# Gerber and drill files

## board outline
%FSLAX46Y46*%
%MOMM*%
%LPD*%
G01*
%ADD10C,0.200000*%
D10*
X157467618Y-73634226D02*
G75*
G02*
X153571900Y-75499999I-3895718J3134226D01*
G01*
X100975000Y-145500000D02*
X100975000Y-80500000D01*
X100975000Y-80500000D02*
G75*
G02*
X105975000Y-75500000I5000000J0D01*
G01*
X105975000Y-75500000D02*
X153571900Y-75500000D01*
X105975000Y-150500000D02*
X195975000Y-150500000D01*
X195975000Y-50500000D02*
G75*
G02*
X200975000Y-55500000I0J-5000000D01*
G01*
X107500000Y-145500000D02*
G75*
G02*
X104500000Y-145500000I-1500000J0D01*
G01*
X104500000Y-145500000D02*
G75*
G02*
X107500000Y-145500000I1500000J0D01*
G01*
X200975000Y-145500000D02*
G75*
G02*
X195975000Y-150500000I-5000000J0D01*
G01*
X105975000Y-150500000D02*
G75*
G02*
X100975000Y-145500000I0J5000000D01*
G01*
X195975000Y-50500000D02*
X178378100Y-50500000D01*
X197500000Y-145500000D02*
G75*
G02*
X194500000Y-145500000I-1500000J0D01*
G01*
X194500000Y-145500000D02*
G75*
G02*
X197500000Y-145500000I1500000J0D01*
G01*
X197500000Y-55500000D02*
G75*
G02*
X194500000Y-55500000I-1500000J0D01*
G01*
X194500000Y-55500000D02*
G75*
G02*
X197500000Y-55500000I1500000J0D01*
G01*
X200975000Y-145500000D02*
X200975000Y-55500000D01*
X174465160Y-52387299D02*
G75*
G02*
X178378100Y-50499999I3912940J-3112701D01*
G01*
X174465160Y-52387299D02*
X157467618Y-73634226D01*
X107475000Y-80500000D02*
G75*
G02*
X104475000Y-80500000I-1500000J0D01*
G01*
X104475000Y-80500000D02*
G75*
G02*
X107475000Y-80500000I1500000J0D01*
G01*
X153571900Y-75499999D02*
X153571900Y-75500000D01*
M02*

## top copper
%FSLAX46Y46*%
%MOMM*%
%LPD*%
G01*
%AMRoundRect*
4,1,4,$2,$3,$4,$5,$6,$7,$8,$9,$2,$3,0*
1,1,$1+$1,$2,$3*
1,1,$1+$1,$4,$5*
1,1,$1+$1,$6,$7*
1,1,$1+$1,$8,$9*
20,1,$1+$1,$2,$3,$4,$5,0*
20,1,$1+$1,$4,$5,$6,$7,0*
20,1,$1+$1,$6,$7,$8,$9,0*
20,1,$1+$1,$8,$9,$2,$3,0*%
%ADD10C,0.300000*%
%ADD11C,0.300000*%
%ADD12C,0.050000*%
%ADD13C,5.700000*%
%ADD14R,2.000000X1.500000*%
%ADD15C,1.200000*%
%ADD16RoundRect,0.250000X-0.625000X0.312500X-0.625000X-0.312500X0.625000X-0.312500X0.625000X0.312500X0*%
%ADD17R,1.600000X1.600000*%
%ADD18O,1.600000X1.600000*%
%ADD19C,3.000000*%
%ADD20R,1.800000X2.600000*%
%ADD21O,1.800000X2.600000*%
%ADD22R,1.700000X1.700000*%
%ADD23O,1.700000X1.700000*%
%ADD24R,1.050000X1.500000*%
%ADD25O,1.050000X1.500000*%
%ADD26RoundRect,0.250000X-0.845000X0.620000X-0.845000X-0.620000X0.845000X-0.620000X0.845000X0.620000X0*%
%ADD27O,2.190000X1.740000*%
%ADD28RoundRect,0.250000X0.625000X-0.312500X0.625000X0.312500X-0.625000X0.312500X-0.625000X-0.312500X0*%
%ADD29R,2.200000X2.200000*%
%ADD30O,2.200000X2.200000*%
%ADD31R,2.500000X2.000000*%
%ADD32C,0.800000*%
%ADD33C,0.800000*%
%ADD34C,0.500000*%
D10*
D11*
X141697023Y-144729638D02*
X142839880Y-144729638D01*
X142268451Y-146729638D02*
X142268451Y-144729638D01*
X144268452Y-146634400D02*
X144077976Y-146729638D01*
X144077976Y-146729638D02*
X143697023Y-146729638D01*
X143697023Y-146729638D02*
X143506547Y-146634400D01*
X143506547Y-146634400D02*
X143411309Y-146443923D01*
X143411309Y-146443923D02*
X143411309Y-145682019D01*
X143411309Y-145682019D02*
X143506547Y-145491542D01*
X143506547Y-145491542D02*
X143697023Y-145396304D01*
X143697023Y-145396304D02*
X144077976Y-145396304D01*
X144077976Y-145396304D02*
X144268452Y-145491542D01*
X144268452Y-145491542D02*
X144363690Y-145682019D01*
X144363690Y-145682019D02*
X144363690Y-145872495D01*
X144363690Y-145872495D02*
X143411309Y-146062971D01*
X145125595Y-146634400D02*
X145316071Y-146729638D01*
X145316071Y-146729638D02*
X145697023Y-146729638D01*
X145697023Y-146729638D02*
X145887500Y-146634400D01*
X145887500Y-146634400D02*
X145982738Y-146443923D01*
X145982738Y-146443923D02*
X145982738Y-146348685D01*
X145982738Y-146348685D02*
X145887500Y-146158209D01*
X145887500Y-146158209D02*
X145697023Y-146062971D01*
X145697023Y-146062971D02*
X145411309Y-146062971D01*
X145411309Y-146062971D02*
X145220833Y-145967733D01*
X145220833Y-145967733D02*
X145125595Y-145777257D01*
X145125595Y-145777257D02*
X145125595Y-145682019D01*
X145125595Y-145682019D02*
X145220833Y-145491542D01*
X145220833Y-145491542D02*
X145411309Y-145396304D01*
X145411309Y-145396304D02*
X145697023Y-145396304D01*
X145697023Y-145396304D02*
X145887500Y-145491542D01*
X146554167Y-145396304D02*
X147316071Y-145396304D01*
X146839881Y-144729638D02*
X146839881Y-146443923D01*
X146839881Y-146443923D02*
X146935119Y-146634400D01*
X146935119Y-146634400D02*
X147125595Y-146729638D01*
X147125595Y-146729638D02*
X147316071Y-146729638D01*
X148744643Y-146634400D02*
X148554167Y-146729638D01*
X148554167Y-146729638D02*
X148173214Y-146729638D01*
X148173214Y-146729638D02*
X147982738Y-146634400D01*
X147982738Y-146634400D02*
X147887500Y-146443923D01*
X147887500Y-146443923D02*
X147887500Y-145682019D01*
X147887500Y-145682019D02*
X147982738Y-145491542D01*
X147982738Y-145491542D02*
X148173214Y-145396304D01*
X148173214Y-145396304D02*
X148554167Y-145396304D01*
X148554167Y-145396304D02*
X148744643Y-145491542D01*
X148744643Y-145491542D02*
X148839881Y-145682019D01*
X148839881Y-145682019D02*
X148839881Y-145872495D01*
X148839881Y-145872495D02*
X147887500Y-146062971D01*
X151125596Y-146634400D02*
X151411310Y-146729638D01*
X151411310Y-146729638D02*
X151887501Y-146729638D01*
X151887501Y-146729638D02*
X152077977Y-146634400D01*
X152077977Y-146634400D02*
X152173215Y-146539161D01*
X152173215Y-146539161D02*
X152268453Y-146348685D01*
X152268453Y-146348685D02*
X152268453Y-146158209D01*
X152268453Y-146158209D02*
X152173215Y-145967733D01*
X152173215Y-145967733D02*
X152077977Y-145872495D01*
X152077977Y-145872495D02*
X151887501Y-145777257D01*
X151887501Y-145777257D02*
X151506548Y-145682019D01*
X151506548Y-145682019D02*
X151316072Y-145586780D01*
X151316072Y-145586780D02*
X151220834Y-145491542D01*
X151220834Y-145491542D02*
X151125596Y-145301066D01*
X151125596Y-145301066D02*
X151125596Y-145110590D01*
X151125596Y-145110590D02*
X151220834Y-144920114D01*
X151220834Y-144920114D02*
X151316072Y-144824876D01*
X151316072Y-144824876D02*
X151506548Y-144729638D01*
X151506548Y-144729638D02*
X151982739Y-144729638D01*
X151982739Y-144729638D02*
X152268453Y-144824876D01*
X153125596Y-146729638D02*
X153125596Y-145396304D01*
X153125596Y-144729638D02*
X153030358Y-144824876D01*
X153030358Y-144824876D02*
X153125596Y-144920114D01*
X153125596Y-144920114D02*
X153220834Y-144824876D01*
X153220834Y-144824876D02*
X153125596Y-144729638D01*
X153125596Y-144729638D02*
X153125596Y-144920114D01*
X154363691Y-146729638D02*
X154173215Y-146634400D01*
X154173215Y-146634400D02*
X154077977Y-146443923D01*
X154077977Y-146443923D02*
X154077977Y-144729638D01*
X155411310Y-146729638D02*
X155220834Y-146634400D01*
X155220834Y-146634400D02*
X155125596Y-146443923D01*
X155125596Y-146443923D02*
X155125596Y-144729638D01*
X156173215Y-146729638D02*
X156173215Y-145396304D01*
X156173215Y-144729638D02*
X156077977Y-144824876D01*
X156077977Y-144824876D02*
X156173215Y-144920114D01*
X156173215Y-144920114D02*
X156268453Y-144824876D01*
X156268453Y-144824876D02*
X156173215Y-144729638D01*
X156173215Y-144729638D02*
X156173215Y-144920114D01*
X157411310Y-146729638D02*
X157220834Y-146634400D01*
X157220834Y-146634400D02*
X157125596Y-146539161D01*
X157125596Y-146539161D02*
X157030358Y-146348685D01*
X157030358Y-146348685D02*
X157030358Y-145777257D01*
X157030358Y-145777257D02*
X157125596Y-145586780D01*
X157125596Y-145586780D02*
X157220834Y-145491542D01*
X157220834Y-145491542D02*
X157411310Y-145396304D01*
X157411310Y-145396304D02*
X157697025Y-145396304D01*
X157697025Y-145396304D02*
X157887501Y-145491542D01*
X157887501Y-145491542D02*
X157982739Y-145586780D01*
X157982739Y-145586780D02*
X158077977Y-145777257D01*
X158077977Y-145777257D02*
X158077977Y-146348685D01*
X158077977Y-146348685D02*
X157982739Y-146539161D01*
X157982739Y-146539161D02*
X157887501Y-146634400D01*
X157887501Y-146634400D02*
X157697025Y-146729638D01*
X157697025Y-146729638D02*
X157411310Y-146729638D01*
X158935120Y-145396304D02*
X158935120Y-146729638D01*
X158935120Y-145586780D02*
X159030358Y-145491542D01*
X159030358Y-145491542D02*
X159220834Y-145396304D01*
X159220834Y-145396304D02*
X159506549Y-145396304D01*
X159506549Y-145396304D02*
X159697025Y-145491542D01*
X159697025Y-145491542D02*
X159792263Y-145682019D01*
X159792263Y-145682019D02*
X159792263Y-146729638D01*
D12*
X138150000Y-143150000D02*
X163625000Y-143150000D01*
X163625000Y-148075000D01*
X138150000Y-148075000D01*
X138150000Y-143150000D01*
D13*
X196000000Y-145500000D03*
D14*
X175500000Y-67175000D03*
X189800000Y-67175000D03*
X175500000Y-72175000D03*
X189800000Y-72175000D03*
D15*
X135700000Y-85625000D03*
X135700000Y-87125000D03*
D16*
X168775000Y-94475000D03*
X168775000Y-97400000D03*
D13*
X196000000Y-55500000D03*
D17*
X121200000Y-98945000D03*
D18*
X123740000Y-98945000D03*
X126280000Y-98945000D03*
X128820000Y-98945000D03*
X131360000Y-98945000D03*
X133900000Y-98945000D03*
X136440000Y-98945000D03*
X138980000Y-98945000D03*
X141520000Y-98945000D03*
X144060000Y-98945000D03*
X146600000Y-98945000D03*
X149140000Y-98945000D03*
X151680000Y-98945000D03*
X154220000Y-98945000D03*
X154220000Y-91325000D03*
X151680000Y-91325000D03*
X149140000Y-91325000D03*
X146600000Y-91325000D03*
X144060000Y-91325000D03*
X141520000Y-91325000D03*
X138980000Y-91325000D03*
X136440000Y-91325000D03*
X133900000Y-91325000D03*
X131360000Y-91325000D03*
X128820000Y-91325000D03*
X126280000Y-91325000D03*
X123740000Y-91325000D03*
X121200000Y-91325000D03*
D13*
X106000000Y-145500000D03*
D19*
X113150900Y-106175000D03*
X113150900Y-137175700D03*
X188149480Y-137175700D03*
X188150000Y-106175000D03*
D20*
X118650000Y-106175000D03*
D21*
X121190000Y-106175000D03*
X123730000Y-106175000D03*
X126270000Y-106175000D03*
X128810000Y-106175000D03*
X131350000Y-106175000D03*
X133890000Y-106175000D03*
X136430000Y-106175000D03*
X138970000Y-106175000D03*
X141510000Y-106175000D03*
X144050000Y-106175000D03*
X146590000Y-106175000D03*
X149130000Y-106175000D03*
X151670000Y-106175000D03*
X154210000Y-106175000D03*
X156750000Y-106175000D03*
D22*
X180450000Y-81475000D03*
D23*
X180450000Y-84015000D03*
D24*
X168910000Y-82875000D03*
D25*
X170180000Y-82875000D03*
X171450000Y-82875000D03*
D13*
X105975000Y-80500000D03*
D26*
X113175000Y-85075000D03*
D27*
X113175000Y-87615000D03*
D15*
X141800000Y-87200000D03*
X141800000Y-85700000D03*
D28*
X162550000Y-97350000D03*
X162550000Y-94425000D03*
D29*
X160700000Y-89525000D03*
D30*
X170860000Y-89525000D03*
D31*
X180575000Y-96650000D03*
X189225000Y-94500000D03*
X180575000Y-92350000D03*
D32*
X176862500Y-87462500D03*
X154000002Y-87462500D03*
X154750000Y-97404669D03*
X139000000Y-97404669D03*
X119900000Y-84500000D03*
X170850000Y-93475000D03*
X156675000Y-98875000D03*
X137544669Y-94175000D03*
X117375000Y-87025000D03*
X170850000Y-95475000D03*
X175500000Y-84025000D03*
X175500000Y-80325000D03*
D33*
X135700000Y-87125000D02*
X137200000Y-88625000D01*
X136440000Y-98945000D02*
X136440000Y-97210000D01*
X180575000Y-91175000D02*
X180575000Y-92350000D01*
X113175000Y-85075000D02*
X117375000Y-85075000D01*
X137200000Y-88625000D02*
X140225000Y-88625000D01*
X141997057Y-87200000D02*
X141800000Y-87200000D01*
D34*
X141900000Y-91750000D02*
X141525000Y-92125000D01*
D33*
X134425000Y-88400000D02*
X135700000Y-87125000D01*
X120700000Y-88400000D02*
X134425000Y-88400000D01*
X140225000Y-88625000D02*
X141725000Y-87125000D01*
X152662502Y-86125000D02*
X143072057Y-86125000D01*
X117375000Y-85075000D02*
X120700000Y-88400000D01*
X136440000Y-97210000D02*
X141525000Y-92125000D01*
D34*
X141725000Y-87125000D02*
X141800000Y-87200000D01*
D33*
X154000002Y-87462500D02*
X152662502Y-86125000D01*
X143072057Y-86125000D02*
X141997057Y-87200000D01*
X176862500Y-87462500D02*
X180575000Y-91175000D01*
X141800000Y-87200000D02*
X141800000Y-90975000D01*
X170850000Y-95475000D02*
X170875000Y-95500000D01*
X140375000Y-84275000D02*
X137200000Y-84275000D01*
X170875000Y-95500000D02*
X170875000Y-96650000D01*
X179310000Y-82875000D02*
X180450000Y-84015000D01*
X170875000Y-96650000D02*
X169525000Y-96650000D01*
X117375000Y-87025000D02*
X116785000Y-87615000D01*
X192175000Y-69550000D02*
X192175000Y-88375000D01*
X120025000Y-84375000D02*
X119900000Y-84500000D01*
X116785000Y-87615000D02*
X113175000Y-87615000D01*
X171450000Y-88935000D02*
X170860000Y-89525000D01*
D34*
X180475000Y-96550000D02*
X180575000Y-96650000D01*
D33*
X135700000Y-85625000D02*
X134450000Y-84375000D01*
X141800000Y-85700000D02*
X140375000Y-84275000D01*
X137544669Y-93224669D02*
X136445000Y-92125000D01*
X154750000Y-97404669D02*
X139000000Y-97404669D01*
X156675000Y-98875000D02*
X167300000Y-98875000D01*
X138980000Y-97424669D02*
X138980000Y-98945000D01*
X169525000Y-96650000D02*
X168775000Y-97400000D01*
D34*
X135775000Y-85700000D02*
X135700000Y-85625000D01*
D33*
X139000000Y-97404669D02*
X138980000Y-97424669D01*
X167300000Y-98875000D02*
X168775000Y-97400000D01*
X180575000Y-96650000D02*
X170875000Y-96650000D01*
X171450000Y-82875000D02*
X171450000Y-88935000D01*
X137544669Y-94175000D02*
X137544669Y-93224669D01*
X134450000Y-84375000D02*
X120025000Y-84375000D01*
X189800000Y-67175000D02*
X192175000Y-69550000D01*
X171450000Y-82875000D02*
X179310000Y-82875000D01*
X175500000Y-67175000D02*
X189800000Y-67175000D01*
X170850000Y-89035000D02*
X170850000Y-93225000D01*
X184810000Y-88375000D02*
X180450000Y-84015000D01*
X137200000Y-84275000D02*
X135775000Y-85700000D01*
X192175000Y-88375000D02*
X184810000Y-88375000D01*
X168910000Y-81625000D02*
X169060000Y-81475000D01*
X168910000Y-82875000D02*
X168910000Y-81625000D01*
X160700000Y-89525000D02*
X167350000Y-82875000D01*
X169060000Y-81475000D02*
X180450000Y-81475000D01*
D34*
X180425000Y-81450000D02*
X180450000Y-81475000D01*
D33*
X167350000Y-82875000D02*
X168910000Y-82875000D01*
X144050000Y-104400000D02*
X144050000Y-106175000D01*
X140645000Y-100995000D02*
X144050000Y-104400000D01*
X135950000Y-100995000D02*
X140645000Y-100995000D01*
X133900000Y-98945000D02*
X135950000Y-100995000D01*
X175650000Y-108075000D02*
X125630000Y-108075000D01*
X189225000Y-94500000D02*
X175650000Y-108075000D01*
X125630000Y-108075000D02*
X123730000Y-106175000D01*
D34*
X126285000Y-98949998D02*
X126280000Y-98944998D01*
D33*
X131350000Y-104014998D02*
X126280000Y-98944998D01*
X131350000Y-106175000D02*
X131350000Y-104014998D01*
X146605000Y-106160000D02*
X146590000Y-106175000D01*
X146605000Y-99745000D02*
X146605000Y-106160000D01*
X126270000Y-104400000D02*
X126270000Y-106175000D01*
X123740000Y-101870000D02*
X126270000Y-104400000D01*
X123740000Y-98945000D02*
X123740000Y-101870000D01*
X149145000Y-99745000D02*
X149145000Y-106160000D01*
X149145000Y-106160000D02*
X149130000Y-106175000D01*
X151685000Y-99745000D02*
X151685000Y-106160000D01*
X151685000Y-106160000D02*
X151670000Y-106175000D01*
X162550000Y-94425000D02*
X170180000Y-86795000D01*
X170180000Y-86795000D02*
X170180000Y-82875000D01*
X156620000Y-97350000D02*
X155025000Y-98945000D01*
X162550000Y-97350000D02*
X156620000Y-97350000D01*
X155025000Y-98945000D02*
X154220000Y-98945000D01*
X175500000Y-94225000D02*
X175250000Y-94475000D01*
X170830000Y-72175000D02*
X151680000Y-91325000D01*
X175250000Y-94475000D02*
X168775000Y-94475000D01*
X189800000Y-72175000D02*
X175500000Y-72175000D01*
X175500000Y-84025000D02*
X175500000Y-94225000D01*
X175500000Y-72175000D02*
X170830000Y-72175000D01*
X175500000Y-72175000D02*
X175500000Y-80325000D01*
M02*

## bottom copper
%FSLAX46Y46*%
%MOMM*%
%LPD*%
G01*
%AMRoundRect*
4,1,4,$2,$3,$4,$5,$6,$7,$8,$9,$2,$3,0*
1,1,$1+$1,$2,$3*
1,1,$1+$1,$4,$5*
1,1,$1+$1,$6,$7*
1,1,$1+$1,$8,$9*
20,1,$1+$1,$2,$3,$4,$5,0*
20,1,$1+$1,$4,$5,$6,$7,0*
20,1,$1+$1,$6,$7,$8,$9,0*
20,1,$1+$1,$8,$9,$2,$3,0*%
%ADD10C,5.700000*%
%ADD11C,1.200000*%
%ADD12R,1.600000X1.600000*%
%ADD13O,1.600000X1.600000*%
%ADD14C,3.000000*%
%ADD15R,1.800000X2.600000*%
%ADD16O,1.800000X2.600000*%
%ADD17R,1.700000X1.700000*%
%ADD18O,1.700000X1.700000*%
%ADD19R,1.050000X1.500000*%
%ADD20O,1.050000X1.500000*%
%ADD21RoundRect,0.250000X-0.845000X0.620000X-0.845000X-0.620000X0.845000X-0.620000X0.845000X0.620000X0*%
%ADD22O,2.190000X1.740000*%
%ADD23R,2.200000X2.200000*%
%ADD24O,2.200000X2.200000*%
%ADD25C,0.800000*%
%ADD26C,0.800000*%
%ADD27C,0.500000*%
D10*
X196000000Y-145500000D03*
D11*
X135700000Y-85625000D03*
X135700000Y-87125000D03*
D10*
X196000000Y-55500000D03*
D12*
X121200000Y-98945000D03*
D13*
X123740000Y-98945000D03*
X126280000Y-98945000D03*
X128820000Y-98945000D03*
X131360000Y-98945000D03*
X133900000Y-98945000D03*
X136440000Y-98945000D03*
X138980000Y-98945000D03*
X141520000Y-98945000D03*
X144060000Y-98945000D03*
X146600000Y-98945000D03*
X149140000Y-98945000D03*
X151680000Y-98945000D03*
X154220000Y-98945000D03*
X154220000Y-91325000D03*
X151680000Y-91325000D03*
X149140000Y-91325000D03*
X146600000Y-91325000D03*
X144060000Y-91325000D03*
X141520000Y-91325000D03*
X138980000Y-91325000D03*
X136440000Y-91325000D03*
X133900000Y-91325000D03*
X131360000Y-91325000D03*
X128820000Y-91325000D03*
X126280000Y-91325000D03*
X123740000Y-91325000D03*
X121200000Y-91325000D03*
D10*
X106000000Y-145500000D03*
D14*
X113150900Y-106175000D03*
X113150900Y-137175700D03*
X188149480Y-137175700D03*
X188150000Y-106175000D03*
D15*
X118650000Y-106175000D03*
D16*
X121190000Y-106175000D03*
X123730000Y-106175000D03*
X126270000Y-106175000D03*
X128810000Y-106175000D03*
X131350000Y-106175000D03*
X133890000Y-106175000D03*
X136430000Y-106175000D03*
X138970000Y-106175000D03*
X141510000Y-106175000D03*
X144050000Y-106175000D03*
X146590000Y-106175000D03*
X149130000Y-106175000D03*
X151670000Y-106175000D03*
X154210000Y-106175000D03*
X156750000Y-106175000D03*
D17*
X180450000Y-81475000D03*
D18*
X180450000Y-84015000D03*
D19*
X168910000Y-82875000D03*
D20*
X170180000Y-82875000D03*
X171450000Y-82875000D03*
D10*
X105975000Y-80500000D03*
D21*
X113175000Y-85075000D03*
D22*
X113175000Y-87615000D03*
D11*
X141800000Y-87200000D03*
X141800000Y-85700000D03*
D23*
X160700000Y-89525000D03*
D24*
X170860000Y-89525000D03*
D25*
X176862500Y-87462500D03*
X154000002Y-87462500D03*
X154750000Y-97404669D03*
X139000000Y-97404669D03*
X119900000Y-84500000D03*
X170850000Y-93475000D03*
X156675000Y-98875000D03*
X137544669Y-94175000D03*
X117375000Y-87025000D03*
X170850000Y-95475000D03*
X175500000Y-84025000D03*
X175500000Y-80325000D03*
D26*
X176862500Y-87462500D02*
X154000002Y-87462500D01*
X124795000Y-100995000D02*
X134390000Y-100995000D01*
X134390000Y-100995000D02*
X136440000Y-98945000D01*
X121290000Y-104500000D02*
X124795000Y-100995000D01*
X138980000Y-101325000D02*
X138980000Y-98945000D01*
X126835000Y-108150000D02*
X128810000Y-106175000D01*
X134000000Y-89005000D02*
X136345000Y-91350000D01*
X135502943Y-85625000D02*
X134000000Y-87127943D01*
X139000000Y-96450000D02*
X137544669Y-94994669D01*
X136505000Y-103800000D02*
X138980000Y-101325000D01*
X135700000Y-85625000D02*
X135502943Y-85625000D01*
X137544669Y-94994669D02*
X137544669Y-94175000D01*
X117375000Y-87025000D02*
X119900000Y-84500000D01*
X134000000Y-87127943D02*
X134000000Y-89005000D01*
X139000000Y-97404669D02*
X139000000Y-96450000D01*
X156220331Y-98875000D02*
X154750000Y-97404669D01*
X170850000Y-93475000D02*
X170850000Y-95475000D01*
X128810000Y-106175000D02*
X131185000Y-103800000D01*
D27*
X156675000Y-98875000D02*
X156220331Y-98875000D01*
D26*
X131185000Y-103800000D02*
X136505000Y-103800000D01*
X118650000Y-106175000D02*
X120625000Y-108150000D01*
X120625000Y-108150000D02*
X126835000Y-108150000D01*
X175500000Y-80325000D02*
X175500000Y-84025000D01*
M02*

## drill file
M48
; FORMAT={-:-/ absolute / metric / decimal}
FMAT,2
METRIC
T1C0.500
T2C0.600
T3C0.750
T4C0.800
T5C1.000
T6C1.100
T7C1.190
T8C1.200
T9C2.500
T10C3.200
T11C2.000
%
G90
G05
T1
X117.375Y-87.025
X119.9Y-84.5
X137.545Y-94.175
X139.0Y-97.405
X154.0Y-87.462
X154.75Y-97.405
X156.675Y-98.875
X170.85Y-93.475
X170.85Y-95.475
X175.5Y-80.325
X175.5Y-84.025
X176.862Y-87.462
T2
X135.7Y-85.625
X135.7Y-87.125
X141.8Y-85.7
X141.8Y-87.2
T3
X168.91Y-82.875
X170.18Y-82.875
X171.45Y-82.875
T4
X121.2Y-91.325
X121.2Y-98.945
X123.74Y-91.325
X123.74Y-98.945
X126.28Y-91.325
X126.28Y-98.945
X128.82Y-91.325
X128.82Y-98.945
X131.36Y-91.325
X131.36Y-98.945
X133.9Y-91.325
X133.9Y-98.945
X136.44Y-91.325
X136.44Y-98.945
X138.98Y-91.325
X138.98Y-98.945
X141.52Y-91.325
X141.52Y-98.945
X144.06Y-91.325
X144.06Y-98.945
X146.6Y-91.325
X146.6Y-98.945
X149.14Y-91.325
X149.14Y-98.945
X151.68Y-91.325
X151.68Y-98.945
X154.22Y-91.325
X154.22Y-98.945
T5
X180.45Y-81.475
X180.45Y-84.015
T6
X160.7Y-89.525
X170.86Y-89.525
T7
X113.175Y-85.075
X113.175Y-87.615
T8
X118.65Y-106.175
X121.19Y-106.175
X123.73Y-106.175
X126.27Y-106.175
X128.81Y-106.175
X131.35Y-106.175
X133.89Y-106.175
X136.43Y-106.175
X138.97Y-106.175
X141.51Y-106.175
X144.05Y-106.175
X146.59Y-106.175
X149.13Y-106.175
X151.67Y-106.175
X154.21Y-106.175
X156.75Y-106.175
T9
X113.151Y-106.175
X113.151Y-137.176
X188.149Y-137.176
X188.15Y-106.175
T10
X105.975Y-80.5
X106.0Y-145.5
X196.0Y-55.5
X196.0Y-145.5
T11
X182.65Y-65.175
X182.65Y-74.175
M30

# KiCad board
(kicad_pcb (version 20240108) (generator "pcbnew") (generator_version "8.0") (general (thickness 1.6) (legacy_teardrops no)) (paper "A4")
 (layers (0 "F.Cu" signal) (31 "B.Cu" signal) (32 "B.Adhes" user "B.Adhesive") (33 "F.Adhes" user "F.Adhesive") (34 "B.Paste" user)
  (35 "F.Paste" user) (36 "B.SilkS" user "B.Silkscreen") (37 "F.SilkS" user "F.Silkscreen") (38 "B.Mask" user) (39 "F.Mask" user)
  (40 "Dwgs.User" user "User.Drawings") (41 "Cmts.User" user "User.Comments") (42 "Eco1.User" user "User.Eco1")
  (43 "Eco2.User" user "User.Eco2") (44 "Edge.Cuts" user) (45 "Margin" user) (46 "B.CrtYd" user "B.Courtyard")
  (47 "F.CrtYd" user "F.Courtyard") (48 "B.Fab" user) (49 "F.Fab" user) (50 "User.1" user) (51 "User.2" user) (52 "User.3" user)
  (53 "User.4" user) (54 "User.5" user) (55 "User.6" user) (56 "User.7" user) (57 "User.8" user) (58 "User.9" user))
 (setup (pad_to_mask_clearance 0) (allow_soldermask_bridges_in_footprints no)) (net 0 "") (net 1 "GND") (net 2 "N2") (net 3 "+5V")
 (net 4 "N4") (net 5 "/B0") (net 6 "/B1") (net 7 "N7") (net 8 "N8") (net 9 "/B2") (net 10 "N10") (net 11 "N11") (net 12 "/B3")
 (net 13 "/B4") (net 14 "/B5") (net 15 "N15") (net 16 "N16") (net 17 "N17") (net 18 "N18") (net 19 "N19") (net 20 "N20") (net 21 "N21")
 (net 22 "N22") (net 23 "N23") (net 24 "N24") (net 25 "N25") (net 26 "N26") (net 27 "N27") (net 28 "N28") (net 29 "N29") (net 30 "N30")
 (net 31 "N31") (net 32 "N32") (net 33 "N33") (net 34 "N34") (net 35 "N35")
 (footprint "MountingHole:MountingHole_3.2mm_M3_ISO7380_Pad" (layer "F.Cu") (at 196 145.5)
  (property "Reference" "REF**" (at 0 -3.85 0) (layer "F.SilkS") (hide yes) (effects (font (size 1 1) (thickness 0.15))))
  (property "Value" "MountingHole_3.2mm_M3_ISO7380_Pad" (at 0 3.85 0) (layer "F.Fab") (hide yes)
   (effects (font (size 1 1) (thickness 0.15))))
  (pad "1" thru_hole circle (at 0 0) (size 5.7 5.7) (drill 3.2) (layers "*.Cu" "*.Mask") (remove_unused_layers no)))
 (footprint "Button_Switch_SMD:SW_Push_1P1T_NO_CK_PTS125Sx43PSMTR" (layer "F.Cu") (at 182.65 69.675)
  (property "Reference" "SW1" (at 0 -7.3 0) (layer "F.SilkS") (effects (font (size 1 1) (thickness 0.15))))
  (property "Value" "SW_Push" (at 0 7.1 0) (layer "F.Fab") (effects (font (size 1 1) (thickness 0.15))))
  (pad "" np_thru_hole circle (at 0 -4.5) (size 2 2) (drill 2) (layers "*.Cu" "*.Mask"))
  (pad "" np_thru_hole circle (at 0 4.5) (size 2 2) (drill 2) (layers "*.Cu" "*.Mask"))
  (pad "1" smd rect (at -7.15 -2.5) (size 2 1.5) (layers "F.Cu" "F.Paste" "F.Mask") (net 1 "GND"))
  (pad "1" smd rect (at 7.15 -2.5) (size 2 1.5) (layers "F.Cu" "F.Paste" "F.Mask") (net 1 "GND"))
  (pad "2" smd rect (at -7.15 2.5) (size 2 1.5) (layers "F.Cu" "F.Paste" "F.Mask") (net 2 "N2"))
  (pad "2" smd rect (at 7.15 2.5) (size 2 1.5) (layers "F.Cu" "F.Paste" "F.Mask") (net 2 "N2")))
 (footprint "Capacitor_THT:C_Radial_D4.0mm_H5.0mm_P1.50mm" (layer "F.Cu") (at 135.7 85.625 -90)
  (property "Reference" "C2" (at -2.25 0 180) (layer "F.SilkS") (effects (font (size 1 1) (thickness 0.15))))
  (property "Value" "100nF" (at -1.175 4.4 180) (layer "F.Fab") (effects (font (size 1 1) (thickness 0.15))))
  (pad "1" thru_hole circle (at 0 0 270) (size 1.2 1.2) (drill 0.6) (layers "*.Cu" "*.Mask") (remove_unused_layers no) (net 1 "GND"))
  (pad "2" thru_hole circle (at 1.5 0 270) (size 1.2 1.2) (drill 0.6) (layers "*.Cu" "*.Mask") (remove_unused_layers no) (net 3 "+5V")))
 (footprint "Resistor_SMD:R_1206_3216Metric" (layer "F.Cu") (at 168.775 95.9375 -90)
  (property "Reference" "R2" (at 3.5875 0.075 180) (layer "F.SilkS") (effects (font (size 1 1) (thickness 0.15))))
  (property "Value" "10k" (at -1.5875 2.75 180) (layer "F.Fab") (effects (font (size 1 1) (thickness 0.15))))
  (pad "1" smd roundrect (at -1.4625 0 270) (size 1.125 1.75) (layers "F.Cu" "F.Paste" "F.Mask") (roundrect_rratio 0.222222) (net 2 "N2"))
  (pad "2" smd roundrect (at 1.4625 0 270) (size 1.125 1.75) (layers "F.Cu" "F.Paste" "F.Mask") (roundrect_rratio 0.222222) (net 1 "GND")))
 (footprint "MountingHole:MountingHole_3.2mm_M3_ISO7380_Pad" (layer "F.Cu") (at 196 55.5)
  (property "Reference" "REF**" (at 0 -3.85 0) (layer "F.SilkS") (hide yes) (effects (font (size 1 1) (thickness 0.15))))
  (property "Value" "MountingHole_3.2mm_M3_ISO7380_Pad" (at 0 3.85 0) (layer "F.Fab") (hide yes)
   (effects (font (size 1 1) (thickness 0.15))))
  (pad "1" thru_hole circle (at 0 0) (size 5.7 5.7) (drill 3.2) (layers "*.Cu" "*.Mask") (remove_unused_layers no)))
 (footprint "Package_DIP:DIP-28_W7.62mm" (layer "F.Cu") (at 121.2 98.945 90)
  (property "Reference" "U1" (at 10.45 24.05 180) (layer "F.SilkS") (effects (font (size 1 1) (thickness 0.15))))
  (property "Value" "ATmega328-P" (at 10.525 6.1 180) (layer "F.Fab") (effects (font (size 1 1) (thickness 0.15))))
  (pad "1" thru_hole rect (at 0 0 90) (size 1.6 1.6) (drill 0.8) (layers "*.Cu" "*.Mask") (remove_unused_layers no) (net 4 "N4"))
  (pad "2" thru_hole oval (at 0 2.54 90) (size 1.6 1.6) (drill 0.8) (layers "*.Cu" "*.Mask") (remove_unused_layers no) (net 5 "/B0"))
  (pad "3" thru_hole oval (at 0 5.08 90) (size 1.6 1.6) (drill 0.8) (layers "*.Cu" "*.Mask") (remove_unused_layers no) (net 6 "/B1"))
  (pad "4" thru_hole oval (at 0 7.62 90) (size 1.6 1.6) (drill 0.8) (layers "*.Cu" "*.Mask") (remove_unused_layers no) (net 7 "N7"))
  (pad "5" thru_hole oval (at 0 10.16 90) (size 1.6 1.6) (drill 0.8) (layers "*.Cu" "*.Mask") (remove_unused_layers no) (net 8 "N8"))
  (pad "6" thru_hole oval (at 0 12.7 90) (size 1.6 1.6) (drill 0.8) (layers "*.Cu" "*.Mask") (remove_unused_layers no) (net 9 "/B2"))
  (pad "7" thru_hole oval (at 0 15.24 90) (size 1.6 1.6) (drill 0.8) (layers "*.Cu" "*.Mask") (remove_unused_layers no) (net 3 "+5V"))
  (pad "8" thru_hole oval (at 0 17.78 90) (size 1.6 1.6) (drill 0.8) (layers "*.Cu" "*.Mask") (remove_unused_layers no) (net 1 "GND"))
  (pad "9" thru_hole oval (at 0 20.32 90) (size 1.6 1.6) (drill 0.8) (layers "*.Cu" "*.Mask") (remove_unused_layers no) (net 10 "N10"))
  (pad "10" thru_hole oval (at 0 22.86 90) (size 1.6 1.6) (drill 0.8) (layers "*.Cu" "*.Mask") (remove_unused_layers no) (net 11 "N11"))
  (pad "11" thru_hole oval (at 0 25.4 90) (size 1.6 1.6) (drill 0.8) (layers "*.Cu" "*.Mask") (remove_unused_layers no) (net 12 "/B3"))
  (pad "12" thru_hole oval (at 0 27.94 90) (size 1.6 1.6) (drill 0.8) (layers "*.Cu" "*.Mask") (remove_unused_layers no) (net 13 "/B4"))
  (pad "13" thru_hole oval (at 0 30.48 90) (size 1.6 1.6) (drill 0.8) (layers "*.Cu" "*.Mask") (remove_unused_layers no) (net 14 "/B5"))
  (pad "14" thru_hole oval (at 0 33.02 90) (size 1.6 1.6) (drill 0.8) (layers "*.Cu" "*.Mask") (remove_unused_layers no) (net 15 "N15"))
  (pad "15" thru_hole oval (at 7.62 33.02 90) (size 1.6 1.6) (drill 0.8) (layers "*.Cu" "*.Mask") (remove_unused_layers no) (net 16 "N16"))
  (pad "16" thru_hole oval (at 7.62 30.48 90) (size 1.6 1.6) (drill 0.8) (layers "*.Cu" "*.Mask") (remove_unused_layers no) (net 2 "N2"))
  (pad "17" thru_hole oval (at 7.62 27.94 90) (size 1.6 1.6) (drill 0.8) (layers "*.Cu" "*.Mask") (remove_unused_layers no) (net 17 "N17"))
  (pad "18" thru_hole oval (at 7.62 25.4 90) (size 1.6 1.6) (drill 0.8) (layers "*.Cu" "*.Mask") (remove_unused_layers no) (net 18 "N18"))
  (pad "19" thru_hole oval (at 7.62 22.86 90) (size 1.6 1.6) (drill 0.8) (layers "*.Cu" "*.Mask") (remove_unused_layers no) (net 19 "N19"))
  (pad "20" thru_hole oval (at 7.62 20.32 90) (size 1.6 1.6) (drill 0.8) (layers "*.Cu" "*.Mask") (remove_unused_layers no) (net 3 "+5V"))
  (pad "21" thru_hole oval (at 7.62 17.78 90) (size 1.6 1.6) (drill 0.8) (layers "*.Cu" "*.Mask") (remove_unused_layers no) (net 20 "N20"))
  (pad "22" thru_hole oval (at 7.62 15.24 90) (size 1.6 1.6) (drill 0.8) (layers "*.Cu" "*.Mask") (remove_unused_layers no) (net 1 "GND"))
  (pad "23" thru_hole oval (at 7.62 12.7 90) (size 1.6 1.6) (drill 0.8) (layers "*.Cu" "*.Mask") (remove_unused_layers no) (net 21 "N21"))
  (pad "24" thru_hole oval (at 7.62 10.16 90) (size 1.6 1.6) (drill 0.8) (layers "*.Cu" "*.Mask") (remove_unused_layers no) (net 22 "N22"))
  (pad "25" thru_hole oval (at 7.62 7.62 90) (size 1.6 1.6) (drill 0.8) (layers "*.Cu" "*.Mask") (remove_unused_layers no) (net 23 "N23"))
  (pad "26" thru_hole oval (at 7.62 5.08 90) (size 1.6 1.6) (drill 0.8) (layers "*.Cu" "*.Mask") (remove_unused_layers no) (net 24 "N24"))
  (pad "27" thru_hole oval (at 7.62 2.54 90) (size 1.6 1.6) (drill 0.8) (layers "*.Cu" "*.Mask") (remove_unused_layers no) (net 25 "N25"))
  (pad "28" thru_hole oval (at 7.62 0 90) (size 1.6 1.6) (drill 0.8) (layers "*.Cu" "*.Mask") (remove_unused_layers no) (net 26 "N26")))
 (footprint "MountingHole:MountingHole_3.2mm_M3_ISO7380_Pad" (layer "F.Cu") (at 106 145.5)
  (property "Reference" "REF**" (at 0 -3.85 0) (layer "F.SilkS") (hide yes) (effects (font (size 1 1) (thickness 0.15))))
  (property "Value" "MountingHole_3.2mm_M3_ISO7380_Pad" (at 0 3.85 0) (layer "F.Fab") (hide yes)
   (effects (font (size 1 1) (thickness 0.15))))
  (pad "1" thru_hole circle (at 0 0) (size 5.7 5.7) (drill 3.2) (layers "*.Cu" "*.Mask") (remove_unused_layers no)))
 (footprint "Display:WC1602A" (layer "F.Cu") (at 118.65 106.175)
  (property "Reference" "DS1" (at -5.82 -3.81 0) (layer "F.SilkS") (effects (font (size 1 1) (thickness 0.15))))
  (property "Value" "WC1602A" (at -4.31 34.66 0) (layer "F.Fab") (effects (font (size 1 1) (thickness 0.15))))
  (pad "" thru_hole circle (at -5.4991 0) (size 3 3) (drill 2.5) (layers "*.Cu" "*.Mask") (remove_unused_layers no))
  (pad "" thru_hole circle (at -5.4991 31.0007) (size 3 3) (drill 2.5) (layers "*.Cu" "*.Mask") (remove_unused_layers no))
  (pad "" thru_hole circle (at 69.49948 31.0007) (size 3 3) (drill 2.5) (layers "*.Cu" "*.Mask") (remove_unused_layers no))
  (pad "" thru_hole circle (at 69.5 0) (size 3 3) (drill 2.5) (layers "*.Cu" "*.Mask") (remove_unused_layers no))
  (pad "1" thru_hole rect (at 0 0) (size 1.8 2.6) (drill 1.2) (layers "*.Cu" "*.Mask") (remove_unused_layers no) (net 1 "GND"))
  (pad "2" thru_hole oval (at 2.54 0) (size 1.8 2.6) (drill 1.2) (layers "*.Cu" "*.Mask") (remove_unused_layers no) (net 3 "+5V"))
  (pad "3" thru_hole oval (at 5.08 0) (size 1.8 2.6) (drill 1.2) (layers "*.Cu" "*.Mask") (remove_unused_layers no) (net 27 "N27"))
  (pad "4" thru_hole oval (at 7.62 0) (size 1.8 2.6) (drill 1.2) (layers "*.Cu" "*.Mask") (remove_unused_layers no) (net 5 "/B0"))
  (pad "5" thru_hole oval (at 10.16 0) (size 1.8 2.6) (drill 1.2) (layers "*.Cu" "*.Mask") (remove_unused_layers no) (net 1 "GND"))
  (pad "6" thru_hole oval (at 12.7 0) (size 1.8 2.6) (drill 1.2) (layers "*.Cu" "*.Mask") (remove_unused_layers no) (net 6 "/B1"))
  (pad "7" thru_hole oval (at 15.24 0) (size 1.8 2.6) (drill 1.2) (layers "*.Cu" "*.Mask") (remove_unused_layers no) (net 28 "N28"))
  (pad "8" thru_hole oval (at 17.78 0) (size 1.8 2.6) (drill 1.2) (layers "*.Cu" "*.Mask") (remove_unused_layers no) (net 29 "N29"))
  (pad "9" thru_hole oval (at 20.32 0) (size 1.8 2.6) (drill 1.2) (layers "*.Cu" "*.Mask") (remove_unused_layers no) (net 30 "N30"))
  (pad "10" thru_hole oval (at 22.86 0) (size 1.8 2.6) (drill 1.2) (layers "*.Cu" "*.Mask") (remove_unused_layers no) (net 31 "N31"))
  (pad "11" thru_hole oval (at 25.4 0) (size 1.8 2.6) (drill 1.2) (layers "*.Cu" "*.Mask") (remove_unused_layers no) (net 9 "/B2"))
  (pad "12" thru_hole oval (at 27.94 0) (size 1.8 2.6) (drill 1.2) (layers "*.Cu" "*.Mask") (remove_unused_layers no) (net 12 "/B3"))
  (pad "13" thru_hole oval (at 30.48 0) (size 1.8 2.6) (drill 1.2) (layers "*.Cu" "*.Mask") (remove_unused_layers no) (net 13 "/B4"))
  (pad "14" thru_hole oval (at 33.02 0) (size 1.8 2.6) (drill 1.2) (layers "*.Cu" "*.Mask") (remove_unused_layers no) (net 14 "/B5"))
  (pad "15" thru_hole oval (at 35.56 0) (size 1.8 2.6) (drill 1.2) (layers "*.Cu" "*.Mask") (remove_unused_layers no) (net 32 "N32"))
  (pad "16" thru_hole oval (at 38.1 0) (size 1.8 2.6) (drill 1.2) (layers "*.Cu" "*.Mask") (remove_unused_layers no) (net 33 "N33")))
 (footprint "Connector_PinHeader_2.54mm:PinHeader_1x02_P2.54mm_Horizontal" (layer "F.Cu") (at 180.45 81.475)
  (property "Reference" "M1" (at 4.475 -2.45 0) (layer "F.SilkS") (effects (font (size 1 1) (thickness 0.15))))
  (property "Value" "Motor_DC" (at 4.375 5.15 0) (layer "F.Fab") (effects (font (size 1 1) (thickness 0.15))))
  (pad "1" thru_hole rect (at 0 0) (size 1.7 1.7) (drill 1) (layers "*.Cu" "*.Mask") (remove_unused_layers no) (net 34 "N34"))
  (pad "2" thru_hole oval (at 0 2.54) (size 1.7 1.7) (drill 1) (layers "*.Cu" "*.Mask") (remove_unused_layers no) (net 1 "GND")))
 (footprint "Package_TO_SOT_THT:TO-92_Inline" (layer "F.Cu") (at 168.91 82.875)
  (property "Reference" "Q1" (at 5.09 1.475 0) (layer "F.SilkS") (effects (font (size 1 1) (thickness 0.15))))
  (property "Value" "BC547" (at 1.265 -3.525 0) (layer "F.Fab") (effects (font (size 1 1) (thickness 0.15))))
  (pad "1" thru_hole rect (at 0 0) (size 1.05 1.5) (drill 0.75) (layers "*.Cu" "*.Mask") (remove_unused_layers no) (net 34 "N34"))
  (pad "2" thru_hole oval (at 1.27 0) (size 1.05 1.5) (drill 0.75) (layers "*.Cu" "*.Mask") (remove_unused_layers no) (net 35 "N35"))
  (pad "3" thru_hole oval (at 2.54 0) (size 1.05 1.5) (drill 0.75) (layers "*.Cu" "*.Mask") (remove_unused_layers no) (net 1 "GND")))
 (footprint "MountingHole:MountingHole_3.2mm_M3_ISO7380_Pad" (layer "F.Cu") (at 105.975 80.5)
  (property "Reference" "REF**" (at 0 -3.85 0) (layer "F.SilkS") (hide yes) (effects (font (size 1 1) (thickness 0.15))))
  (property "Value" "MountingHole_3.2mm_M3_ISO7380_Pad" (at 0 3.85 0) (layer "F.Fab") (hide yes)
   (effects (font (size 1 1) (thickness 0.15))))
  (pad "1" thru_hole circle (at 0 0) (size 5.7 5.7) (drill 3.2) (layers "*.Cu" "*.Mask") (remove_unused_layers no)))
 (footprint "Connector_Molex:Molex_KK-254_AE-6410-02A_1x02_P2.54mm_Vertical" (layer "F.Cu") (at 113.175 85.075 -90)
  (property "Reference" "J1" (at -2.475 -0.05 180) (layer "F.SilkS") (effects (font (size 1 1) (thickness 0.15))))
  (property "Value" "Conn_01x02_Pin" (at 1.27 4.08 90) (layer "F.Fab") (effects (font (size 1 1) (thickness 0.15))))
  (pad "1" thru_hole roundrect (at 0 0 270) (size 1.74 2.19) (drill 1.19) (layers "*.Cu" "*.Mask") (remove_unused_layers no)
   (roundrect_rratio 0.143678) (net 3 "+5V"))
  (pad "2" thru_hole oval (at 2.54 0 270) (size 1.74 2.19) (drill 1.19) (layers "*.Cu" "*.Mask") (remove_unused_layers no) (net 1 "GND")))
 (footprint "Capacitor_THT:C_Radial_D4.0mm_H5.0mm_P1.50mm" (layer "F.Cu") (at 141.8 87.2 90)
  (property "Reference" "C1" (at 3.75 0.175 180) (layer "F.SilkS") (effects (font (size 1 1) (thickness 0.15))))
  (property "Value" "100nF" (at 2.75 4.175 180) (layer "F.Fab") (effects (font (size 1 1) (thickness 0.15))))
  (pad "1" thru_hole circle (at 0 0 90) (size 1.2 1.2) (drill 0.6) (layers "*.Cu" "*.Mask") (remove_unused_layers no) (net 3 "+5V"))
  (pad "2" thru_hole circle (at 1.5 0 90) (size 1.2 1.2) (drill 0.6) (layers "*.Cu" "*.Mask") (remove_unused_layers no) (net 1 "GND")))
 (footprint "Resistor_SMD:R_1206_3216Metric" (layer "F.Cu") (at 162.55 95.8875 90)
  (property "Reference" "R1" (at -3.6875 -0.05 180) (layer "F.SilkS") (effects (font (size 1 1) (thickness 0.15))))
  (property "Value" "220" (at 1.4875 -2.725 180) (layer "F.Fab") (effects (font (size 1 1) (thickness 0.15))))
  (pad "1" smd roundrect (at -1.4625 0 90) (size 1.125 1.75) (layers "F.Cu" "F.Paste" "F.Mask") (roundrect_rratio 0.222222) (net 15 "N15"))
  (pad "2" smd roundrect (at 1.4625 0 90) (size 1.125 1.75) (layers "F.Cu" "F.Paste" "F.Mask") (roundrect_rratio 0.222222) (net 35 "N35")))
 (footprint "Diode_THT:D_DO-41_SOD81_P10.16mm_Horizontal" (layer "F.Cu") (at 160.7 89.525)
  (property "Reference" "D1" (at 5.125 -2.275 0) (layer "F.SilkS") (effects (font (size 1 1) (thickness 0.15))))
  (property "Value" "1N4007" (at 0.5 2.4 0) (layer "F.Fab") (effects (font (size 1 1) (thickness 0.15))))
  (pad "1" thru_hole rect (at 0 0) (size 2.2 2.2) (drill 1.1) (layers "*.Cu" "*.Mask") (remove_unused_layers no) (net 34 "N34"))
  (pad "2" thru_hole oval (at 10.16 0) (size 2.2 2.2) (drill 1.1) (layers "*.Cu" "*.Mask") (remove_unused_layers no) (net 1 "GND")))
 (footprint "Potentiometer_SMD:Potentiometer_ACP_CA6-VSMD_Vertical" (layer "F.Cu") (at 184.9 94.5)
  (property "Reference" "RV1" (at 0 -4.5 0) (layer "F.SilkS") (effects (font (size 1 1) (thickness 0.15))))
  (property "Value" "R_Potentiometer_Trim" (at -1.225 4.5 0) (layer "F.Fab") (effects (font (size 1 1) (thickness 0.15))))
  (pad "1" smd rect (at -4.325 2.15) (size 2.5 2) (layers "F.Cu" "F.Paste" "F.Mask") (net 1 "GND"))
  (pad "2" smd rect (at 4.325 0) (size 2.5 2) (layers "F.Cu" "F.Paste" "F.Mask") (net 27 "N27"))
  (pad "3" smd rect (at -4.325 -2.15) (size 2.5 2) (layers "F.Cu" "F.Paste" "F.Mask") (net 3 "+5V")))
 (gr_arc (start 157.467618 73.634226) (mid 155.73163 75.009497) (end 153.5719 75.499999) (stroke (width 0.2) (type default))
  (layer "Edge.Cuts"))
 (gr_line (start 100.975 145.5) (end 100.975 80.5) (stroke (width 0.2) (type default)) (layer "Edge.Cuts"))
 (gr_arc (start 100.975 80.5) (mid 102.439466 76.964466) (end 105.975 75.5) (stroke (width 0.2) (type default)) (layer "Edge.Cuts"))
 (gr_line (start 105.975 75.5) (end 153.5719 75.5) (stroke (width 0.2) (type default)) (layer "Edge.Cuts"))
 (gr_line (start 105.975 150.5) (end 195.975 150.5) (stroke (width 0.2) (type default)) (layer "Edge.Cuts"))
 (gr_arc (start 195.975 50.5) (mid 199.510534 51.964466) (end 200.975 55.5) (stroke (width 0.2) (type default)) (layer "Edge.Cuts"))
 (gr_circle (center 106 145.5) (end 107.5 145.5) (stroke (width 0.2) (type default)) (fill none) (layer "Edge.Cuts"))
 (gr_arc (start 200.975 145.5) (mid 199.510534 149.035534) (end 195.975 150.5) (stroke (width 0.2) (type default)) (layer "Edge.Cuts"))
 (gr_arc (start 105.975 150.5) (mid 102.439466 149.035534) (end 100.975 145.5) (stroke (width 0.2) (type default)) (layer "Edge.Cuts"))
 (gr_line (start 195.975 50.5) (end 178.3781 50.5) (stroke (width 0.2) (type default)) (layer "Edge.Cuts"))
 (gr_circle (center 196 145.5) (end 197.5 145.5) (stroke (width 0.2) (type default)) (fill none) (layer "Edge.Cuts"))
 (gr_circle (center 196 55.5) (end 197.5 55.5) (stroke (width 0.2) (type default)) (fill none) (layer "Edge.Cuts"))
 (gr_line (start 200.975 145.5) (end 200.975 55.5) (stroke (width 0.2) (type default)) (layer "Edge.Cuts"))
 (gr_arc (start 174.46516 52.387299) (mid 176.205947 50.996473) (end 178.3781 50.5) (stroke (width 0.2) (type default)) (layer "Edge.Cuts"))
 (gr_line (start 174.46516 52.387299) (end 157.467618 73.634226) (stroke (width 0.2) (type default)) (layer "Edge.Cuts"))
 (gr_circle (center 105.975 80.5) (end 107.475 80.5) (stroke (width 0.2) (type default)) (fill none) (layer "Edge.Cuts"))
 (gr_line (start 153.5719 75.499999) (end 153.5719 75.5) (stroke (width 0.2) (type default)) (layer "Edge.Cuts"))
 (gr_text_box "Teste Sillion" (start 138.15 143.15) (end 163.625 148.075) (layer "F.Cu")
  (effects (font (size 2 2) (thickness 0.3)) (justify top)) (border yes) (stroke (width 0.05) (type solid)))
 (segment (start 135.7 87.125) (end 137.2 88.625) (width 0.8) (layer "F.Cu") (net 3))
 (segment (start 136.44 98.945) (end 136.44 97.21) (width 0.8) (layer "F.Cu") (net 3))
 (segment (start 180.575 91.175) (end 180.575 92.35) (width 0.8) (layer "F.Cu") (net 3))
 (segment (start 113.175 85.075) (end 117.375 85.075) (width 0.8) (layer "F.Cu") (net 3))
 (segment (start 137.2 88.625) (end 140.225 88.625) (width 0.8) (layer "F.Cu") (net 3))
 (segment (start 141.997057 87.2) (end 141.8 87.2) (width 0.8) (layer "F.Cu") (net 3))
 (segment (start 141.9 91.75) (end 141.525 92.125) (width 0.5) (layer "F.Cu") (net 3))
 (segment (start 134.425 88.4) (end 135.7 87.125) (width 0.8) (layer "F.Cu") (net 3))
 (segment (start 120.7 88.4) (end 134.425 88.4) (width 0.8) (layer "F.Cu") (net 3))
 (segment (start 140.225 88.625) (end 141.725 87.125) (width 0.8) (layer "F.Cu") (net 3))
 (segment (start 152.662502 86.125) (end 143.072057 86.125) (width 0.8) (layer "F.Cu") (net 3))
 (segment (start 117.375 85.075) (end 120.7 88.4) (width 0.8) (layer "F.Cu") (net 3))
 (segment (start 136.44 97.21) (end 141.525 92.125) (width 0.8) (layer "F.Cu") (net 3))
 (segment (start 141.725 87.125) (end 141.8 87.2) (width 0.5) (layer "F.Cu") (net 3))
 (segment (start 154.000002 87.4625) (end 152.662502 86.125) (width 0.8) (layer "F.Cu") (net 3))
 (segment (start 143.072057 86.125) (end 141.997057 87.2) (width 0.8) (layer "F.Cu") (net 3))
 (segment (start 176.8625 87.4625) (end 180.575 91.175) (width 0.8) (layer "F.Cu") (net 3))
 (segment (start 141.8 87.2) (end 141.8 90.975) (width 0.8) (layer "F.Cu") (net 3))
 (via (at 176.8625 87.4625) (size 0.8) (drill 0.5) (layers "F.Cu" "B.Cu") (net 3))
 (via (at 154.000002 87.4625) (size 0.8) (drill 0.5) (layers "F.Cu" "B.Cu") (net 3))
 (segment (start 176.8625 87.4625) (end 154.000002 87.4625) (width 0.8) (layer "B.Cu") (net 3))
 (segment (start 124.795 100.995) (end 134.39 100.995) (width 0.8) (layer "B.Cu") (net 3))
 (segment (start 134.39 100.995) (end 136.44 98.945) (width 0.8) (layer "B.Cu") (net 3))
 (segment (start 121.29 104.5) (end 124.795 100.995) (width 0.8) (layer "B.Cu") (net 3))
 (segment (start 170.85 95.475) (end 170.875 95.5) (width 0.8) (layer "F.Cu") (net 1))
 (segment (start 140.375 84.275) (end 137.2 84.275) (width 0.8) (layer "F.Cu") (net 1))
 (segment (start 170.875 95.5) (end 170.875 96.65) (width 0.8) (layer "F.Cu") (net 1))
 (segment (start 179.31 82.875) (end 180.45 84.015) (width 0.8) (layer "F.Cu") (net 1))
 (segment (start 170.875 96.65) (end 169.525 96.65) (width 0.8) (layer "F.Cu") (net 1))
 (segment (start 117.375 87.025) (end 116.785 87.615) (width 0.8) (layer "F.Cu") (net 1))
 (segment (start 192.175 69.55) (end 192.175 88.375) (width 0.8) (layer "F.Cu") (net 1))
 (segment (start 120.025 84.375) (end 119.9 84.5) (width 0.8) (layer "F.Cu") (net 1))
 (segment (start 116.785 87.615) (end 113.175 87.615) (width 0.8) (layer "F.Cu") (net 1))
 (segment (start 171.45 88.935) (end 170.86 89.525) (width 0.8) (layer "F.Cu") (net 1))
 (segment (start 180.475 96.55) (end 180.575 96.65) (width 0.5) (layer "F.Cu") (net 1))
 (segment (start 135.7 85.625) (end 134.45 84.375) (width 0.8) (layer "F.Cu") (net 1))
 (segment (start 141.8 85.7) (end 140.375 84.275) (width 0.8) (layer "F.Cu") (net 1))
 (segment (start 137.544669 93.224669) (end 136.445 92.125) (width 0.8) (layer "F.Cu") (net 1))
 (segment (start 154.75 97.404669) (end 139 97.404669) (width 0.8) (layer "F.Cu") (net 1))
 (segment (start 156.675 98.875) (end 167.3 98.875) (width 0.8) (layer "F.Cu") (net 1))
 (segment (start 138.98 97.424669) (end 138.98 98.945) (width 0.8) (layer "F.Cu") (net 1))
 (segment (start 169.525 96.65) (end 168.775 97.4) (width 0.8) (layer "F.Cu") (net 1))
 (segment (start 135.775 85.7) (end 135.7 85.625) (width 0.5) (layer "F.Cu") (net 1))
 (segment (start 139 97.404669) (end 138.98 97.424669) (width 0.8) (layer "F.Cu") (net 1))
 (segment (start 167.3 98.875) (end 168.775 97.4) (width 0.8) (layer "F.Cu") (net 1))
 (segment (start 180.575 96.65) (end 170.875 96.65) (width 0.8) (layer "F.Cu") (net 1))
 (segment (start 171.45 82.875) (end 171.45 88.935) (width 0.8) (layer "F.Cu") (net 1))
 (segment (start 137.544669 94.175) (end 137.544669 93.224669) (width 0.8) (layer "F.Cu") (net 1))
 (segment (start 134.45 84.375) (end 120.025 84.375) (width 0.8) (layer "F.Cu") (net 1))
 (segment (start 189.8 67.175) (end 192.175 69.55) (width 0.8) (layer "F.Cu") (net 1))
 (segment (start 171.45 82.875) (end 179.31 82.875) (width 0.8) (layer "F.Cu") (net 1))
 (segment (start 175.5 67.175) (end 189.8 67.175) (width 0.8) (layer "F.Cu") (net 1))
 (segment (start 170.85 89.035) (end 170.85 93.225) (width 0.8) (layer "F.Cu") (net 1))
 (segment (start 184.81 88.375) (end 180.45 84.015) (width 0.8) (layer "F.Cu") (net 1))
 (segment (start 137.2 84.275) (end 135.775 85.7) (width 0.8) (layer "F.Cu") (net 1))
 (segment (start 192.175 88.375) (end 184.81 88.375) (width 0.8) (layer "F.Cu") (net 1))
 (via (at 154.75 97.404669) (size 0.8) (drill 0.5) (layers "F.Cu" "B.Cu") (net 1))
 (via (at 139 97.404669) (size 0.8) (drill 0.5) (layers "F.Cu" "B.Cu") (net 1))
 (via (at 119.9 84.5) (size 0.8) (drill 0.5) (layers "F.Cu" "B.Cu") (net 1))
 (via (at 170.85 93.475) (size 0.8) (drill 0.5) (layers "F.Cu" "B.Cu") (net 1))
 (via (at 156.675 98.875) (size 0.8) (drill 0.5) (layers "F.Cu" "B.Cu") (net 1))
 (via (at 137.544669 94.175) (size 0.8) (drill 0.5) (layers "F.Cu" "B.Cu") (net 1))
 (via (at 117.375 87.025) (size 0.8) (drill 0.5) (layers "F.Cu" "B.Cu") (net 1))
 (via (at 170.85 95.475) (size 0.8) (drill 0.5) (layers "F.Cu" "B.Cu") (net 1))
 (segment (start 138.98 101.325) (end 138.98 98.945) (width 0.8) (layer "B.Cu") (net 1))
 (segment (start 126.835 108.15) (end 128.81 106.175) (width 0.8) (layer "B.Cu") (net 1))
 (segment (start 134 89.005) (end 136.345 91.35) (width 0.8) (layer "B.Cu") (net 1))
 (segment (start 135.502943 85.625) (end 134 87.127943) (width 0.8) (layer "B.Cu") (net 1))
 (segment (start 139 96.45) (end 137.544669 94.994669) (width 0.8) (layer "B.Cu") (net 1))
 (segment (start 136.505 103.8) (end 138.98 101.325) (width 0.8) (layer "B.Cu") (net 1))
 (segment (start 135.7 85.625) (end 135.502943 85.625) (width 0.8) (layer "B.Cu") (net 1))
 (segment (start 137.544669 94.994669) (end 137.544669 94.175) (width 0.8) (layer "B.Cu") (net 1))
 (segment (start 117.375 87.025) (end 119.9 84.5) (width 0.8) (layer "B.Cu") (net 1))
 (segment (start 134 87.127943) (end 134 89.005) (width 0.8) (layer "B.Cu") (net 1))
 (segment (start 139 97.404669) (end 139 96.45) (width 0.8) (layer "B.Cu") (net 1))
 (segment (start 156.220331 98.875) (end 154.75 97.404669) (width 0.8) (layer "B.Cu") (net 1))
 (segment (start 170.85 93.475) (end 170.85 95.475) (width 0.8) (layer "B.Cu") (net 1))
 (segment (start 128.81 106.175) (end 131.185 103.8) (width 0.8) (layer "B.Cu") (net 1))
 (segment (start 156.675 98.875) (end 156.220331 98.875) (width 0.5) (layer "B.Cu") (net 1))
 (segment (start 131.185 103.8) (end 136.505 103.8) (width 0.8) (layer "B.Cu") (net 1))
 (segment (start 118.65 106.175) (end 120.625 108.15) (width 0.8) (layer "B.Cu") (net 1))
 (segment (start 120.625 108.15) (end 126.835 108.15) (width 0.8) (layer "B.Cu") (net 1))
 (segment (start 168.91 81.625) (end 169.06 81.475) (width 0.8) (layer "F.Cu") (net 34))
 (segment (start 168.91 82.875) (end 168.91 81.625) (width 0.8) (layer "F.Cu") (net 34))
 (segment (start 160.7 89.525) (end 167.35 82.875) (width 0.8) (layer "F.Cu") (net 34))
 (segment (start 169.06 81.475) (end 180.45 81.475) (width 0.8) (layer "F.Cu") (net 34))
 (segment (start 180.425 81.45) (end 180.45 81.475) (width 0.5) (layer "F.Cu") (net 34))
 (segment (start 167.35 82.875) (end 168.91 82.875) (width 0.8) (layer "F.Cu") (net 34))
 (segment (start 144.05 104.4) (end 144.05 106.175) (width 0.8) (layer "F.Cu") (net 9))
 (segment (start 140.645 100.995) (end 144.05 104.4) (width 0.8) (layer "F.Cu") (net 9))
 (segment (start 135.95 100.995) (end 140.645 100.995) (width 0.8) (layer "F.Cu") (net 9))
 (segment (start 133.9 98.945) (end 135.95 100.995) (width 0.8) (layer "F.Cu") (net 9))
 (segment (start 175.65 108.075) (end 125.63 108.075) (width 0.8) (layer "F.Cu") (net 27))
 (segment (start 189.225 94.5) (end 175.65 108.075) (width 0.8) (layer "F.Cu") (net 27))
 (segment (start 125.63 108.075) (end 123.73 106.175) (width 0.8) (layer "F.Cu") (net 27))
 (segment (start 126.285 98.949998) (end 126.28 98.944998) (width 0.5) (layer "F.Cu") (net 6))
 (segment (start 131.35 104.014998) (end 126.28 98.944998) (width 0.8) (layer "F.Cu") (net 6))
 (segment (start 131.35 106.175) (end 131.35 104.014998) (width 0.8) (layer "F.Cu") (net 6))
 (segment (start 146.605 106.16) (end 146.59 106.175) (width 0.8) (layer "F.Cu") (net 12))
 (segment (start 146.605 99.745) (end 146.605 106.16) (width 0.8) (layer "F.Cu") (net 12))
 (segment (start 126.27 104.4) (end 126.27 106.175) (width 0.8) (layer "F.Cu") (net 5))
 (segment (start 123.74 101.87) (end 126.27 104.4) (width 0.8) (layer "F.Cu") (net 5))
 (segment (start 123.74 98.945) (end 123.74 101.87) (width 0.8) (layer "F.Cu") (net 5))
 (segment (start 149.145 99.745) (end 149.145 106.16) (width 0.8) (layer "F.Cu") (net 13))
 (segment (start 149.145 106.16) (end 149.13 106.175) (width 0.8) (layer "F.Cu") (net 13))
 (segment (start 151.685 99.745) (end 151.685 106.16) (width 0.8) (layer "F.Cu") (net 14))
 (segment (start 151.685 106.16) (end 151.67 106.175) (width 0.8) (layer "F.Cu") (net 14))
 (segment (start 162.55 94.425) (end 170.18 86.795) (width 0.8) (layer "F.Cu") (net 35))
 (segment (start 170.18 86.795) (end 170.18 82.875) (width 0.8) (layer "F.Cu") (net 35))
 (segment (start 156.62 97.35) (end 155.025 98.945) (width 0.8) (layer "F.Cu") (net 15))
 (segment (start 162.55 97.35) (end 156.62 97.35) (width 0.8) (layer "F.Cu") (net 15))
 (segment (start 155.025 98.945) (end 154.22 98.945) (width 0.8) (layer "F.Cu") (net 15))
 (segment (start 175.5 94.225) (end 175.25 94.475) (width 0.8) (layer "F.Cu") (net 2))
 (segment (start 170.83 72.175) (end 151.68 91.325) (width 0.8) (layer "F.Cu") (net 2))
 (segment (start 175.25 94.475) (end 168.775 94.475) (width 0.8) (layer "F.Cu") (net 2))
 (segment (start 189.8 72.175) (end 175.5 72.175) (width 0.8) (layer "F.Cu") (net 2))
 (segment (start 175.5 84.025) (end 175.5 94.225) (width 0.8) (layer "F.Cu") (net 2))
 (segment (start 175.5 72.175) (end 170.83 72.175) (width 0.8) (layer "F.Cu") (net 2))
 (segment (start 175.5 72.175) (end 175.5 80.325) (width 0.8) (layer "F.Cu") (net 2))
 (via (at 175.5 84.025) (size 0.8) (drill 0.5) (layers "F.Cu" "B.Cu") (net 2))
 (via (at 175.5 80.325) (size 0.8) (drill 0.5) (layers "F.Cu" "B.Cu") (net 2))
 (segment (start 175.5 80.325) (end 175.5 84.025) (width 0.8) (layer "B.Cu") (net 2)))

